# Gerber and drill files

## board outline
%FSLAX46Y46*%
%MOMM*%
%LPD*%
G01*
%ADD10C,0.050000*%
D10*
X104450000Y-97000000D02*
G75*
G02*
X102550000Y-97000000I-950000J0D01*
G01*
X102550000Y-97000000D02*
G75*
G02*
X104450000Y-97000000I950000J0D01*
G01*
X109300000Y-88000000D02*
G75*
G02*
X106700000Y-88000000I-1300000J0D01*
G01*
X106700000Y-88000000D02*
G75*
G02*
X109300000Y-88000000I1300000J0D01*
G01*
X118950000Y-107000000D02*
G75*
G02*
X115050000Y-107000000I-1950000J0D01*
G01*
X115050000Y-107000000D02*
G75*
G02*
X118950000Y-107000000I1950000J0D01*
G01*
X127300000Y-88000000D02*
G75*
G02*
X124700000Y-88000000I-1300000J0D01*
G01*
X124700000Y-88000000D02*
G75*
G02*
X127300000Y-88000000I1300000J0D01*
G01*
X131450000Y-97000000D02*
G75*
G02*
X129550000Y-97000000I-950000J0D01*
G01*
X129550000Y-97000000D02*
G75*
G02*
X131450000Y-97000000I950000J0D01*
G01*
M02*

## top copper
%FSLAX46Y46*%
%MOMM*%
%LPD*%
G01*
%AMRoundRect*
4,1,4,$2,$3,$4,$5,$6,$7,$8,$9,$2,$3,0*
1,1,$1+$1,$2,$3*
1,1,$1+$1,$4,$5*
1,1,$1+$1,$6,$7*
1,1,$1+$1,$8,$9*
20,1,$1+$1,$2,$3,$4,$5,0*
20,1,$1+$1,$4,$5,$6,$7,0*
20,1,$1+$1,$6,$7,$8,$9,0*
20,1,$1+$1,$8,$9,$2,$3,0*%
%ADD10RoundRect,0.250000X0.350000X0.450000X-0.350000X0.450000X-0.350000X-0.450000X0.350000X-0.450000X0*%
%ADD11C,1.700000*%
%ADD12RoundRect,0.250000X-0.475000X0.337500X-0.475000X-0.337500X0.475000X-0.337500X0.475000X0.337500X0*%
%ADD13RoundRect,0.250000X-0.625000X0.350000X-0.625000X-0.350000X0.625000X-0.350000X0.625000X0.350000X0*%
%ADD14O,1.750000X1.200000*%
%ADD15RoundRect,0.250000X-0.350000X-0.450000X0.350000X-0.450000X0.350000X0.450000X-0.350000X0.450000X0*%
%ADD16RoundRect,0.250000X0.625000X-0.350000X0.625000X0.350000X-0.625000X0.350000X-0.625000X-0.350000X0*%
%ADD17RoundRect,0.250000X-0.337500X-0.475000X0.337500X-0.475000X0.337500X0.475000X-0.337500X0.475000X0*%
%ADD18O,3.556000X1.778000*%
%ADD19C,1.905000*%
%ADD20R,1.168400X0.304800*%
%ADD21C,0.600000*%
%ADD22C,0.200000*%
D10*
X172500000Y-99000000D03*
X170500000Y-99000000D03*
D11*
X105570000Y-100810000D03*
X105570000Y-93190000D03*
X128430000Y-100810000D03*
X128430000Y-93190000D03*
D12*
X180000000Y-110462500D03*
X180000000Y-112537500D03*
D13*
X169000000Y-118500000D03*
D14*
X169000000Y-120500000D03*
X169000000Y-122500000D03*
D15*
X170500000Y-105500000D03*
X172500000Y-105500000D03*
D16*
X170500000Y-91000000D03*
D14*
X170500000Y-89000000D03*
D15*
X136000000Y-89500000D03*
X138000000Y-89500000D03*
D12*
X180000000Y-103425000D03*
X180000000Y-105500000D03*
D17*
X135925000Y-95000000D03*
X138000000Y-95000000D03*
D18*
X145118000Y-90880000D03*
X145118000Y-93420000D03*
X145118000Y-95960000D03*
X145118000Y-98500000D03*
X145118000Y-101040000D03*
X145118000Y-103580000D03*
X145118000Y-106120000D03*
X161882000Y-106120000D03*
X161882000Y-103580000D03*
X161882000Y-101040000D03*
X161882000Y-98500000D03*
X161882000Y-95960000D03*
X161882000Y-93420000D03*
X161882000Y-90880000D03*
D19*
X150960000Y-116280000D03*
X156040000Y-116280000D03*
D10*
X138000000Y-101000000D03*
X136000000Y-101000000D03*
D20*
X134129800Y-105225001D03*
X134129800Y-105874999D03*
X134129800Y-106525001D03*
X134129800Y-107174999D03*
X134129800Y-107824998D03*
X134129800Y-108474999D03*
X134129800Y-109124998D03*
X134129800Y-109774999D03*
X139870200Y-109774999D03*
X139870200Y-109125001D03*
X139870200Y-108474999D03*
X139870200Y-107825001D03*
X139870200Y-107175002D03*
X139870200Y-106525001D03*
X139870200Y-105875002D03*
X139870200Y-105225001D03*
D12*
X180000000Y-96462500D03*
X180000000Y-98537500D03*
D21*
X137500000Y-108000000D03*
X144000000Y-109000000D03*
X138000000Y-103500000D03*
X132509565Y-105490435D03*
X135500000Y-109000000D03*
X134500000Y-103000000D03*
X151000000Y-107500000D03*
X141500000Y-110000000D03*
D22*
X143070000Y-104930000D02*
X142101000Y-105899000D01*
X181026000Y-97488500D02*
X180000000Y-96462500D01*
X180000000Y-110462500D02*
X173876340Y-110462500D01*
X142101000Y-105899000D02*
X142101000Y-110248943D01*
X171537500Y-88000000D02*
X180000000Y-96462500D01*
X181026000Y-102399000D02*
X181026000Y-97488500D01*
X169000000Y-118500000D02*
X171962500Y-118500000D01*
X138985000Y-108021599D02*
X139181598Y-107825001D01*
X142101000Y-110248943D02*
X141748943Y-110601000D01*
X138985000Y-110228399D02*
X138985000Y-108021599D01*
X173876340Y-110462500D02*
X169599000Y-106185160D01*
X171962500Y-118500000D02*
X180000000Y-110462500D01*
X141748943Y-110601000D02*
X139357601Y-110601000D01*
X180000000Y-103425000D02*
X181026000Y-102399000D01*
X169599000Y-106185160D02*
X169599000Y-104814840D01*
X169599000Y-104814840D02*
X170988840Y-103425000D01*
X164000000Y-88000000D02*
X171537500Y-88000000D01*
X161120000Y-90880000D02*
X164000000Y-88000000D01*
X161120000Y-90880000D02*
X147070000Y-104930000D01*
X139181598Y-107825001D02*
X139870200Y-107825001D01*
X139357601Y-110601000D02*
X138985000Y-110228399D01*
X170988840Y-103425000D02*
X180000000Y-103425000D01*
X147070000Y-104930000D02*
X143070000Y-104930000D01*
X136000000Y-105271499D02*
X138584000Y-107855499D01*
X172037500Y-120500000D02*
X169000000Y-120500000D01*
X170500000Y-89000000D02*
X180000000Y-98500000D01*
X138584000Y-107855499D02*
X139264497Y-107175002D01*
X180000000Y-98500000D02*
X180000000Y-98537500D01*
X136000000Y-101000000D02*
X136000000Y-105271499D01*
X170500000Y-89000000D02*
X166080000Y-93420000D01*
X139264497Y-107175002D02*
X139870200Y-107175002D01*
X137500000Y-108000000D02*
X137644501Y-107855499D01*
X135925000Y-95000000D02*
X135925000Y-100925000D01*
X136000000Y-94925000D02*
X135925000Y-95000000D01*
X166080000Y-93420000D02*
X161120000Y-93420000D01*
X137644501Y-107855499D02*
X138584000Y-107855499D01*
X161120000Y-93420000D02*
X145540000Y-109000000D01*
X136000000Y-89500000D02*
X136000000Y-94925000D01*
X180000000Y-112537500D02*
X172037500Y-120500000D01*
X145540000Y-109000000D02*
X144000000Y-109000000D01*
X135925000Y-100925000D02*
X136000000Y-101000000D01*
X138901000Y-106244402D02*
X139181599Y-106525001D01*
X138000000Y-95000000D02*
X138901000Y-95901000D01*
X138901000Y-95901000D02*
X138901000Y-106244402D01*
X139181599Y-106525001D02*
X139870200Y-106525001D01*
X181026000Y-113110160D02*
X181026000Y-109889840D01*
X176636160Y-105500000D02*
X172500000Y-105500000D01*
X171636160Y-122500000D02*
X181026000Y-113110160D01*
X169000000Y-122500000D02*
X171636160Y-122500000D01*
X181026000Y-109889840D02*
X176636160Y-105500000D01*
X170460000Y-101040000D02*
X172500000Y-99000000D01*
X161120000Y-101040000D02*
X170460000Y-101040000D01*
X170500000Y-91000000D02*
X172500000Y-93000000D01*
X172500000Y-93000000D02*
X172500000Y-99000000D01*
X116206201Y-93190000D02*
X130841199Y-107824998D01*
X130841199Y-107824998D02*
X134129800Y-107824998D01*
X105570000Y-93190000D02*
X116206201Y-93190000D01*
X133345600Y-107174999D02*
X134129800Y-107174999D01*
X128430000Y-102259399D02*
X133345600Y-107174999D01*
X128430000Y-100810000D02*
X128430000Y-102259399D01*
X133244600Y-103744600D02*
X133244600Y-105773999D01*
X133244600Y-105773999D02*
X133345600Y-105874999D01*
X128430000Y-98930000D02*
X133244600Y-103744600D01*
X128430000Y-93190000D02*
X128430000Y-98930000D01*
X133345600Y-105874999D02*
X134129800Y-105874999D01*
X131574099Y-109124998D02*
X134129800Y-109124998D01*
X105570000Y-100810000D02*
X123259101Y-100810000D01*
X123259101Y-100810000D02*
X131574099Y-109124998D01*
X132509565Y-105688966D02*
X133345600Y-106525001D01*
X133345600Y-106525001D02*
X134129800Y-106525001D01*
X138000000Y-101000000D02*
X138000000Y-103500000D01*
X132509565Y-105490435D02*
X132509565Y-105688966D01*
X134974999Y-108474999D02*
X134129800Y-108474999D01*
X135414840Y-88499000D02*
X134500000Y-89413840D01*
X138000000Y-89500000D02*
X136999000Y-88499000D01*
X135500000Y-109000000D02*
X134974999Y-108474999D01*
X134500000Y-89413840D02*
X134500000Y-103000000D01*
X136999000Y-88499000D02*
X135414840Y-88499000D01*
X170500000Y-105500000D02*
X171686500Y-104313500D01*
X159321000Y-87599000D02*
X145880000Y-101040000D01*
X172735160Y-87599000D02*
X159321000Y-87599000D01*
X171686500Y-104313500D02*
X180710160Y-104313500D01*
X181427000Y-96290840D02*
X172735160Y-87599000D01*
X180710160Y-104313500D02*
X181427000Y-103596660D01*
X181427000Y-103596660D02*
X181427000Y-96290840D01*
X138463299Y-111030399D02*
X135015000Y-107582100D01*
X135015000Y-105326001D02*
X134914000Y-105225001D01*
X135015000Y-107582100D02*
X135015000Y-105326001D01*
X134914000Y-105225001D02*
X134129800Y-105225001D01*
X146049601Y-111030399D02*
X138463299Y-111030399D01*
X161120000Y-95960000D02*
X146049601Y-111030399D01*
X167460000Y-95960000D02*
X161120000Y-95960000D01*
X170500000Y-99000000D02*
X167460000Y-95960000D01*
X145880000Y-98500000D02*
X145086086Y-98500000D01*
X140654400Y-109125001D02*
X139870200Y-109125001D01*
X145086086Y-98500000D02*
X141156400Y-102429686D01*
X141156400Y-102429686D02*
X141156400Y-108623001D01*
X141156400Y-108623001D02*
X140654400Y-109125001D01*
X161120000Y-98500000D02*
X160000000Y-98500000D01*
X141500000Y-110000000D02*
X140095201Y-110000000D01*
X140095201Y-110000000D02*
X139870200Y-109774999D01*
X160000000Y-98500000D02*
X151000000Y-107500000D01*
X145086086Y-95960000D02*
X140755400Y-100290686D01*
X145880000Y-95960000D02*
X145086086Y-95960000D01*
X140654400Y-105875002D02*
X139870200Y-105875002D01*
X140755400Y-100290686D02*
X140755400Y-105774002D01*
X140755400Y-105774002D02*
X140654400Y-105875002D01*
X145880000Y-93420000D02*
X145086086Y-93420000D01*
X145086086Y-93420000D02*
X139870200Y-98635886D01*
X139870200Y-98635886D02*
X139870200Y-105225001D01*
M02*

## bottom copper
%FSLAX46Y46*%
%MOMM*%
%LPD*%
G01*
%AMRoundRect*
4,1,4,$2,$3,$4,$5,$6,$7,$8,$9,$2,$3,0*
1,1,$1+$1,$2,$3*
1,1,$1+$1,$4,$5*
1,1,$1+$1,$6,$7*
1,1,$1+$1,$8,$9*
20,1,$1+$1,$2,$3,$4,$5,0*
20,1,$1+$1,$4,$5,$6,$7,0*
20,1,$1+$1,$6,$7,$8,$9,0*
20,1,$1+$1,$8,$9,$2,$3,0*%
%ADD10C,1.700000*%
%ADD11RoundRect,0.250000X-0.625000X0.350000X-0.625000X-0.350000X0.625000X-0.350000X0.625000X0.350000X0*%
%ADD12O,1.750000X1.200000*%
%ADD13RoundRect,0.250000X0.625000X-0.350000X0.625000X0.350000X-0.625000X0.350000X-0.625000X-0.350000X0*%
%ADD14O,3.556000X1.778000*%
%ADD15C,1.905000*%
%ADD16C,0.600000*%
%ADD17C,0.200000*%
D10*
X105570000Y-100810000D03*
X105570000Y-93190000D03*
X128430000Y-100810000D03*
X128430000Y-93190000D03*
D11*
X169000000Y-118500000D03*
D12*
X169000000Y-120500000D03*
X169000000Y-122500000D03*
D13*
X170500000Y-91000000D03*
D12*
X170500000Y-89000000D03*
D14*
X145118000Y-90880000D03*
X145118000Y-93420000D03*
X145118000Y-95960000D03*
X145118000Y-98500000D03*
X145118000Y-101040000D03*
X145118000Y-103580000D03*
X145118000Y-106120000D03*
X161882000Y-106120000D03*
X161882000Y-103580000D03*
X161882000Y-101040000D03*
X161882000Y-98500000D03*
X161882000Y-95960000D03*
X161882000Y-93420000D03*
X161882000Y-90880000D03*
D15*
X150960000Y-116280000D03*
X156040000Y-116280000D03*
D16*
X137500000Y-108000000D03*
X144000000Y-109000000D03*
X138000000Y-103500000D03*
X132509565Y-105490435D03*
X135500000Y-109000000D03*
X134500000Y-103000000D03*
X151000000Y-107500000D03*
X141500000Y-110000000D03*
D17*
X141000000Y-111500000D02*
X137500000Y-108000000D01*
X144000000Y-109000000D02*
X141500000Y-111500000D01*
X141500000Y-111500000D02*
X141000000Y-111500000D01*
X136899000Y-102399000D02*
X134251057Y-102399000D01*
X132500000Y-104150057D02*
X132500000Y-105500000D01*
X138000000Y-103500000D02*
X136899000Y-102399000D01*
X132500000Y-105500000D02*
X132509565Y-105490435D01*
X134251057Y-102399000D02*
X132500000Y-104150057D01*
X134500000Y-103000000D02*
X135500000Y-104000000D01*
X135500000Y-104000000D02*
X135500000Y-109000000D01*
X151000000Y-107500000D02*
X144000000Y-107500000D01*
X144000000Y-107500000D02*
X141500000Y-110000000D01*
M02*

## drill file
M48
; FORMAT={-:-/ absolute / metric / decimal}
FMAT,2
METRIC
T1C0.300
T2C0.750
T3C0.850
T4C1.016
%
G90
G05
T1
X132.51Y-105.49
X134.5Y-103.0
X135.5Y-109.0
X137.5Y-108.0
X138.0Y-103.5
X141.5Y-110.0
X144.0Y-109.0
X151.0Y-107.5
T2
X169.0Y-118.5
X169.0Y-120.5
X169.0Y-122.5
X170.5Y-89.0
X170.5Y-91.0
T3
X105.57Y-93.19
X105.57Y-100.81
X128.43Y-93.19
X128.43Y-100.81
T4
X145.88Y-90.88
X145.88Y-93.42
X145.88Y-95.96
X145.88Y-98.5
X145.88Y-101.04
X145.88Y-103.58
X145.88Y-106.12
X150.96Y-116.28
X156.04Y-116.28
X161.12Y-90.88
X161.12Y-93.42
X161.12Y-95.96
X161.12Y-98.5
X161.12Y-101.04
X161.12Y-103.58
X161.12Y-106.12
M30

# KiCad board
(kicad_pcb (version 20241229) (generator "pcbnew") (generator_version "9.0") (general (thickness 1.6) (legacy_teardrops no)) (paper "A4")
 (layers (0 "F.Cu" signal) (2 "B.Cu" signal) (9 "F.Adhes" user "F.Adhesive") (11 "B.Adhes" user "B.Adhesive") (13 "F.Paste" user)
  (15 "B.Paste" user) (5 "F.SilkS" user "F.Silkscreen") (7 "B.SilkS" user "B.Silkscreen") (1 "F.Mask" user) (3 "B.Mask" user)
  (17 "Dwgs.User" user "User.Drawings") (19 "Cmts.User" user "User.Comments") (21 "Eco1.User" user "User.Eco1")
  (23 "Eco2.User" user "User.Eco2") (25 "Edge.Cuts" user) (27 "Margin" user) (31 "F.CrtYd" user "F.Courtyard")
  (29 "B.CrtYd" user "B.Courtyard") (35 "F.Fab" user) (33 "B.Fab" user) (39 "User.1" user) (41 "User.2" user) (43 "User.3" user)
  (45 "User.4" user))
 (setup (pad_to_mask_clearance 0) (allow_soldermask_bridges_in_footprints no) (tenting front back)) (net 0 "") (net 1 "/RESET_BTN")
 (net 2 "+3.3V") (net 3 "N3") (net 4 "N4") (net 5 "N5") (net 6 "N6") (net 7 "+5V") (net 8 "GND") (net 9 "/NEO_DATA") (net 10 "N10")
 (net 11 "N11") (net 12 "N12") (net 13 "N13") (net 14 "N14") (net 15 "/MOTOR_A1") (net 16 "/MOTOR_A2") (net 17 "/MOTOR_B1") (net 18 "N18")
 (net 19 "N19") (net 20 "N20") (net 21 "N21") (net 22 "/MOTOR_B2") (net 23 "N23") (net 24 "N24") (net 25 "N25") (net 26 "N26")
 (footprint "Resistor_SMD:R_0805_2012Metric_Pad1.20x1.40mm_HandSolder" (layer "F.Cu") (at 171.5 99 180)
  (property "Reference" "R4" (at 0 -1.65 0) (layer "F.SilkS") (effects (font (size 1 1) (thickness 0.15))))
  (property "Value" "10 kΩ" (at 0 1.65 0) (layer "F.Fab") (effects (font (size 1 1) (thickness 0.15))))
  (pad "1" smd roundrect (at -1 0 180) (size 1.2 1.4) (layers "F.Cu" "F.Mask" "F.Paste") (roundrect_rratio 0.208333) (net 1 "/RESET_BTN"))
  (pad "2" smd roundrect (at 1 0 180) (size 1.2 1.4) (layers "F.Cu" "F.Mask" "F.Paste") (roundrect_rratio 0.208333) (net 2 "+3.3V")))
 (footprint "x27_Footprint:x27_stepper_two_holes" (layer "F.Cu") (at 114.46 86.84 180)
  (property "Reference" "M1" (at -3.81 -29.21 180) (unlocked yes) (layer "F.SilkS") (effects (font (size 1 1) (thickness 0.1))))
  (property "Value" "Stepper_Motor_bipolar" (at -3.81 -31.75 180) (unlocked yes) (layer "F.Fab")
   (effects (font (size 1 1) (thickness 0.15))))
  (fp_circle (center 10.96 -10.16) (end 11.91 -10.16) (stroke (width 0.05) (type default)) (fill no) (layer "Edge.Cuts"))
  (fp_circle (center 6.46 -1.16) (end 7.76 -1.16) (stroke (width 0.05) (type default)) (fill no) (layer "Edge.Cuts"))
  (fp_circle (center -2.54 -20.16) (end -0.59 -20.16) (stroke (width 0.05) (type default)) (fill no) (layer "Edge.Cuts"))
  (fp_circle (center -11.54 -1.16) (end -10.24 -1.16) (stroke (width 0.05) (type default)) (fill no) (layer "Edge.Cuts"))
  (fp_circle (center -16.04 -10.16) (end -15.09 -10.16) (stroke (width 0.05) (type default)) (fill no) (layer "Edge.Cuts"))
  (pad "1" thru_hole circle (at 8.89 -13.97 180) (size 1.7 1.7) (drill 0.85) (layers "*.Cu" "*.Mask") (remove_unused_layers no) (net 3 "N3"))
  (pad "2" thru_hole circle (at 8.89 -6.35 180) (size 1.7 1.7) (drill 0.85) (layers "*.Cu" "*.Mask") (remove_unused_layers no) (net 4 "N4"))
  (pad "3" thru_hole circle (at -13.97 -13.97 180) (size 1.7 1.7) (drill 0.85) (layers "*.Cu" "*.Mask") (remove_unused_layers no)
   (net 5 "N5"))
  (pad "4" thru_hole circle (at -13.97 -6.35 180) (size 1.7 1.7) (drill 0.85) (layers "*.Cu" "*.Mask") (remove_unused_layers no)
   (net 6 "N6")))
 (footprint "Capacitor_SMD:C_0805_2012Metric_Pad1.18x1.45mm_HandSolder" (layer "F.Cu") (at 180 111.5 -90)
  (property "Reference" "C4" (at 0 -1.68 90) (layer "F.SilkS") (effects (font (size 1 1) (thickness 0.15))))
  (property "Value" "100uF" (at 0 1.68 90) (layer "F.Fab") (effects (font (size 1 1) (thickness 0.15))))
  (pad "1" smd roundrect (at -1.0375 0 270) (size 1.175 1.45) (layers "F.Cu" "F.Mask" "F.Paste") (roundrect_rratio 0.212766) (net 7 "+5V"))
  (pad "2" smd roundrect (at 1.0375 0 270) (size 1.175 1.45) (layers "F.Cu" "F.Mask" "F.Paste") (roundrect_rratio 0.212766) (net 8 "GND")))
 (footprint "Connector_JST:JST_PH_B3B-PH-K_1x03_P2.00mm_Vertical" (layer "F.Cu") (at 169 118.5 -90)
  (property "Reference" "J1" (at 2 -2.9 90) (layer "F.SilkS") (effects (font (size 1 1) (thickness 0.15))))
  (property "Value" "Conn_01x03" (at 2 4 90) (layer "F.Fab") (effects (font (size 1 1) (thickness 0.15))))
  (pad "1" thru_hole roundrect (at 0 0 270) (size 1.2 1.75) (drill 0.75) (layers "*.Cu" "*.Mask") (remove_unused_layers no)
   (roundrect_rratio 0.208333) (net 7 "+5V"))
  (pad "2" thru_hole oval (at 2 0 270) (size 1.2 1.75) (drill 0.75) (layers "*.Cu" "*.Mask") (remove_unused_layers no) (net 8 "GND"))
  (pad "3" thru_hole oval (at 4 0 270) (size 1.2 1.75) (drill 0.75) (layers "*.Cu" "*.Mask") (remove_unused_layers no) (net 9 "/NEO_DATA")))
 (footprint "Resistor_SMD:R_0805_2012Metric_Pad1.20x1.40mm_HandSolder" (layer "F.Cu") (at 171.5 105.5)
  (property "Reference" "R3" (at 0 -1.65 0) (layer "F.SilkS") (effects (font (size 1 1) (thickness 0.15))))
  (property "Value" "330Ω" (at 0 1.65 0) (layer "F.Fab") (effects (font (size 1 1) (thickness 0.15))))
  (pad "1" smd roundrect (at -1 0) (size 1.2 1.4) (layers "F.Cu" "F.Mask" "F.Paste") (roundrect_rratio 0.208333) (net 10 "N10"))
  (pad "2" smd roundrect (at 1 0) (size 1.2 1.4) (layers "F.Cu" "F.Mask" "F.Paste") (roundrect_rratio 0.208333) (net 9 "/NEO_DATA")))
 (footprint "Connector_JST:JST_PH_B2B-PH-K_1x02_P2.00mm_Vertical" (layer "F.Cu") (at 170.5 91 90)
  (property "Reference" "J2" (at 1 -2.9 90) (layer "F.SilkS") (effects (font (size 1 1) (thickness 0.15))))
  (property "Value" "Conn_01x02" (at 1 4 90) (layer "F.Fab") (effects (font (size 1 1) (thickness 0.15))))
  (pad "1" thru_hole roundrect (at 0 0 90) (size 1.2 1.75) (drill 0.75) (layers "*.Cu" "*.Mask") (remove_unused_layers no)
   (roundrect_rratio 0.208333) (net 1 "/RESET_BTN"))
  (pad "2" thru_hole oval (at 2 0 90) (size 1.2 1.75) (drill 0.75) (layers "*.Cu" "*.Mask") (remove_unused_layers no) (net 8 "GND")))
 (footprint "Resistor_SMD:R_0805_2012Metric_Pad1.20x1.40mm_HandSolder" (layer "F.Cu") (at 137 89.5)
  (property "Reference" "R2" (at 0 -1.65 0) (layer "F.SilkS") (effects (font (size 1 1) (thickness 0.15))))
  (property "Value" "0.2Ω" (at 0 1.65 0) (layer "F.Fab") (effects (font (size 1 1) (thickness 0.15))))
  (pad "1" smd roundrect (at -1 0) (size 1.2 1.4) (layers "F.Cu" "F.Mask" "F.Paste") (roundrect_rratio 0.208333) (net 8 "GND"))
  (pad "2" smd roundrect (at 1 0) (size 1.2 1.4) (layers "F.Cu" "F.Mask" "F.Paste") (roundrect_rratio 0.208333) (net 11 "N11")))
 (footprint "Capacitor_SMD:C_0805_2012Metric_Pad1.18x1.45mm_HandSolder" (layer "F.Cu") (at 180 104.4625 -90)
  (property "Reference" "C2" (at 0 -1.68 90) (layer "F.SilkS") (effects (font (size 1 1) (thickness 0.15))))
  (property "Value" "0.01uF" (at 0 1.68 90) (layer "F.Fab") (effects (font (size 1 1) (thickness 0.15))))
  (pad "1" smd roundrect (at -1.0375 0 270) (size 1.175 1.45) (layers "F.Cu" "F.Mask" "F.Paste") (roundrect_rratio 0.212766) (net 7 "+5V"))
  (pad "2" smd roundrect (at 1.0375 0 270) (size 1.175 1.45) (layers "F.Cu" "F.Mask" "F.Paste") (roundrect_rratio 0.212766) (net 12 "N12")))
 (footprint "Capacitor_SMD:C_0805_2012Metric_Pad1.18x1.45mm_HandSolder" (layer "F.Cu") (at 136.9625 95)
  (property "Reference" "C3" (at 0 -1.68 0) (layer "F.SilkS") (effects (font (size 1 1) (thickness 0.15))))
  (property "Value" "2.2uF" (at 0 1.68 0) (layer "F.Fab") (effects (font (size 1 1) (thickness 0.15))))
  (pad "1" smd roundrect (at -1.0375 0) (size 1.175 1.45) (layers "F.Cu" "F.Mask" "F.Paste") (roundrect_rratio 0.212766) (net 8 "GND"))
  (pad "2" smd roundrect (at 1.0375 0) (size 1.175 1.45) (layers "F.Cu" "F.Mask" "F.Paste") (roundrect_rratio 0.212766) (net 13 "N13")))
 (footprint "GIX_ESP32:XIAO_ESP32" (layer "F.Cu") (at 153.5 98.5)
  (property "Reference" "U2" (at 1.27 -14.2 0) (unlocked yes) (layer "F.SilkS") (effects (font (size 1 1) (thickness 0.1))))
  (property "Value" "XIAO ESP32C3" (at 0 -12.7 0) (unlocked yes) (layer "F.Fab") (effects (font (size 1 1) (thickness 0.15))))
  (pad "1" thru_hole oval (at -7.62 -7.62) (size 3.556 1.778) (drill 1.016 (offset -0.762 0)) (layers "*.Cu" "*.Mask")
   (remove_unused_layers no) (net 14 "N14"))
  (pad "2" thru_hole oval (at -7.62 -5.08) (size 3.556 1.778) (drill 1.016 (offset -0.762 0)) (layers "*.Cu" "*.Mask")
   (remove_unused_layers no) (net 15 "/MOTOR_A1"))
  (pad "3" thru_hole oval (at -7.62 -2.54) (size 3.556 1.778) (drill 1.016 (offset -0.762 0)) (layers "*.Cu" "*.Mask")
   (remove_unused_layers no) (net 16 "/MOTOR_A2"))
  (pad "4" thru_hole oval (at -7.62 0) (size 3.556 1.778) (drill 1.016 (offset -0.762 0)) (layers "*.Cu" "*.Mask") (remove_unused_layers no)
   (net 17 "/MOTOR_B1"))
  (pad "5" thru_hole oval (at -7.62 2.54) (size 3.556 1.778) (drill 1.016 (offset -0.762 0)) (layers "*.Cu" "*.Mask")
   (remove_unused_layers no) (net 10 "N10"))
  (pad "6" thru_hole oval (at -7.62 5.08) (size 3.556 1.778) (drill 1.016 (offset -0.762 0)) (layers "*.Cu" "*.Mask")
   (remove_unused_layers no) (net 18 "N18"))
  (pad "7" thru_hole oval (at -7.62 7.62) (size 3.556 1.778) (drill 1.016 (offset -0.762 0)) (layers "*.Cu" "*.Mask")
   (remove_unused_layers no) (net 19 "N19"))
  (pad "8" thru_hole oval (at 7.62 7.62) (size 3.556 1.778) (drill 1.016 (offset 0.762 0)) (layers "*.Cu" "*.Mask")
   (remove_unused_layers no) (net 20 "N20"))
  (pad "9" thru_hole oval (at 7.62 5.08) (size 3.556 1.778) (drill 1.016 (offset 0.762 0)) (layers "*.Cu" "*.Mask")
   (remove_unused_layers no) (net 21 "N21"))
  (pad "10" thru_hole oval (at 7.62 2.54) (size 3.556 1.778) (drill 1.016 (offset 0.762 0)) (layers "*.Cu" "*.Mask")
   (remove_unused_layers no) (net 1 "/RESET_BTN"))
  (pad "11" thru_hole oval (at 7.62 0) (size 3.556 1.778) (drill 1.016 (offset 0.762 0)) (layers "*.Cu" "*.Mask") (remove_unused_layers no)
   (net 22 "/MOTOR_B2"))
  (pad "12" thru_hole oval (at 7.62 -2.54) (size 3.556 1.778) (drill 1.016 (offset 0.762 0)) (layers "*.Cu" "*.Mask")
   (remove_unused_layers no) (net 2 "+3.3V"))
  (pad "13" thru_hole oval (at 7.62 -5.08) (size 3.556 1.778) (drill 1.016 (offset 0.762 0)) (layers "*.Cu" "*.Mask")
   (remove_unused_layers no) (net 8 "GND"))
  (pad "14" thru_hole oval (at 7.62 -7.62) (size 3.556 1.778) (drill 1.016 (offset 0.762 0)) (layers "*.Cu" "*.Mask")
   (remove_unused_layers no) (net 7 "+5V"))
  (pad "15" thru_hole circle (at -2.54 17.78) (size 1.905 1.905) (drill 1.016) (layers "*.Cu" "*.Mask") (remove_unused_layers no)
   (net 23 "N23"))
  (pad "16" thru_hole circle (at 2.54 17.78) (size 1.905 1.905) (drill 1.016) (layers "*.Cu" "*.Mask") (remove_unused_layers no)
   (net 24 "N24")))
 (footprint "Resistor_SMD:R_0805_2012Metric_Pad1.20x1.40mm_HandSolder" (layer "F.Cu") (at 137 101 180)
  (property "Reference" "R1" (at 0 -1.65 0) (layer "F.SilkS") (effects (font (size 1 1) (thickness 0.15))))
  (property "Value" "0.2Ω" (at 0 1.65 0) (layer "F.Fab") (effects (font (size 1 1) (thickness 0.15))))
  (pad "1" smd roundrect (at -1 0 180) (size 1.2 1.4) (layers "F.Cu" "F.Mask" "F.Paste") (roundrect_rratio 0.208333) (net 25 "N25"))
  (pad "2" smd roundrect (at 1 0 180) (size 1.2 1.4) (layers "F.Cu" "F.Mask" "F.Paste") (roundrect_rratio 0.208333) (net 8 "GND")))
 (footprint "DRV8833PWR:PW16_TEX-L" (layer "F.Cu") (at 137 107.5)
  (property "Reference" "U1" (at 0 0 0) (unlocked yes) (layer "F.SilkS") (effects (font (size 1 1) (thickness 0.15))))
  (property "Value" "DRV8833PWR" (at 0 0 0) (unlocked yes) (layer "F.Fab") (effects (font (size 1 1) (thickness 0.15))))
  (pad "1" smd rect (at -2.8702 -2.274999) (size 1.1684 0.3048) (layers "F.Cu" "F.Mask" "F.Paste") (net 2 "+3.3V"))
  (pad "2" smd rect (at -2.8702 -1.625001) (size 1.1684 0.3048) (layers "F.Cu" "F.Mask" "F.Paste") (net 6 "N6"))
  (pad "3" smd rect (at -2.8702 -0.974999) (size 1.1684 0.3048) (layers "F.Cu" "F.Mask" "F.Paste") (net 25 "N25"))
  (pad "4" smd rect (at -2.8702 -0.325001) (size 1.1684 0.3048) (layers "F.Cu" "F.Mask" "F.Paste") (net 5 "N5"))
  (pad "5" smd rect (at -2.8702 0.324998) (size 1.1684 0.3048) (layers "F.Cu" "F.Mask" "F.Paste") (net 4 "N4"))
  (pad "6" smd rect (at -2.8702 0.974999) (size 1.1684 0.3048) (layers "F.Cu" "F.Mask" "F.Paste") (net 11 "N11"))
  (pad "7" smd rect (at -2.8702 1.624998) (size 1.1684 0.3048) (layers "F.Cu" "F.Mask" "F.Paste") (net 3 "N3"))
  (pad "8" smd rect (at -2.8702 2.274999) (size 1.1684 0.3048) (layers "F.Cu" "F.Mask" "F.Paste") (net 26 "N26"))
  (pad "9" smd rect (at 2.8702 2.274999) (size 1.1684 0.3048) (layers "F.Cu" "F.Mask" "F.Paste") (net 22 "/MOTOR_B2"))
  (pad "10" smd rect (at 2.8702 1.625001) (size 1.1684 0.3048) (layers "F.Cu" "F.Mask" "F.Paste") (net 17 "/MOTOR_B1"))
  (pad "11" smd rect (at 2.8702 0.974999) (size 1.1684 0.3048) (layers "F.Cu" "F.Mask" "F.Paste") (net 12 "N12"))
  (pad "12" smd rect (at 2.8702 0.325001) (size 1.1684 0.3048) (layers "F.Cu" "F.Mask" "F.Paste") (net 7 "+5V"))
  (pad "13" smd rect (at 2.8702 -0.324998) (size 1.1684 0.3048) (layers "F.Cu" "F.Mask" "F.Paste") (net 8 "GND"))
  (pad "14" smd rect (at 2.8702 -0.974999) (size 1.1684 0.3048) (layers "F.Cu" "F.Mask" "F.Paste") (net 13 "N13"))
  (pad "15" smd rect (at 2.8702 -1.624998) (size 1.1684 0.3048) (layers "F.Cu" "F.Mask" "F.Paste") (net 16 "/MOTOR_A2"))
  (pad "16" smd rect (at 2.8702 -2.274999) (size 1.1684 0.3048) (layers "F.Cu" "F.Mask" "F.Paste") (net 15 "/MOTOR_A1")))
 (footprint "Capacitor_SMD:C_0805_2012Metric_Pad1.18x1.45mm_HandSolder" (layer "F.Cu") (at 180 97.5 -90)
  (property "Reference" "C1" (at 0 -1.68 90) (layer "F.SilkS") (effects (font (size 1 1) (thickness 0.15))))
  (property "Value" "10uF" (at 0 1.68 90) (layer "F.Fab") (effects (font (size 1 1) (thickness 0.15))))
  (pad "1" smd roundrect (at -1.0375 0 270) (size 1.175 1.45) (layers "F.Cu" "F.Mask" "F.Paste") (roundrect_rratio 0.212766) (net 7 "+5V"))
  (pad "2" smd roundrect (at 1.0375 0 270) (size 1.175 1.45) (layers "F.Cu" "F.Mask" "F.Paste") (roundrect_rratio 0.212766) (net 8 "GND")))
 (segment (start 143.07 104.93) (end 142.101 105.899) (width 0.2) (layer "F.Cu") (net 7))
 (segment (start 181.026 97.4885) (end 180 96.4625) (width 0.2) (layer "F.Cu") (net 7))
 (segment (start 180 110.4625) (end 173.87634 110.4625) (width 0.2) (layer "F.Cu") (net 7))
 (segment (start 142.101 105.899) (end 142.101 110.248943) (width 0.2) (layer "F.Cu") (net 7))
 (segment (start 171.5375 88) (end 180 96.4625) (width 0.2) (layer "F.Cu") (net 7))
 (segment (start 181.026 102.399) (end 181.026 97.4885) (width 0.2) (layer "F.Cu") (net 7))
 (segment (start 169 118.5) (end 171.9625 118.5) (width 0.2) (layer "F.Cu") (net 7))
 (segment (start 138.985 108.021599) (end 139.181598 107.825001) (width 0.2) (layer "F.Cu") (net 7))
 (segment (start 142.101 110.248943) (end 141.748943 110.601) (width 0.2) (layer "F.Cu") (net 7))
 (segment (start 138.985 110.228399) (end 138.985 108.021599) (width 0.2) (layer "F.Cu") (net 7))
 (segment (start 173.87634 110.4625) (end 169.599 106.18516) (width 0.2) (layer "F.Cu") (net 7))
 (segment (start 171.9625 118.5) (end 180 110.4625) (width 0.2) (layer "F.Cu") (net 7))
 (segment (start 141.748943 110.601) (end 139.357601 110.601) (width 0.2) (layer "F.Cu") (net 7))
 (segment (start 180 103.425) (end 181.026 102.399) (width 0.2) (layer "F.Cu") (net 7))
 (segment (start 169.599 106.18516) (end 169.599 104.81484) (width 0.2) (layer "F.Cu") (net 7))
 (segment (start 169.599 104.81484) (end 170.98884 103.425) (width 0.2) (layer "F.Cu") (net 7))
 (segment (start 164 88) (end 171.5375 88) (width 0.2) (layer "F.Cu") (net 7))
 (segment (start 161.12 90.88) (end 164 88) (width 0.2) (layer "F.Cu") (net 7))
 (segment (start 161.12 90.88) (end 147.07 104.93) (width 0.2) (layer "F.Cu") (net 7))
 (segment (start 139.181598 107.825001) (end 139.8702 107.825001) (width 0.2) (layer "F.Cu") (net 7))
 (segment (start 139.357601 110.601) (end 138.985 110.228399) (width 0.2) (layer "F.Cu") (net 7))
 (segment (start 170.98884 103.425) (end 180 103.425) (width 0.2) (layer "F.Cu") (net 7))
 (segment (start 147.07 104.93) (end 143.07 104.93) (width 0.2) (layer "F.Cu") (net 7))
 (segment (start 136 105.271499) (end 138.584 107.855499) (width 0.2) (layer "F.Cu") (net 8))
 (segment (start 172.0375 120.5) (end 169 120.5) (width 0.2) (layer "F.Cu") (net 8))
 (segment (start 170.5 89) (end 180 98.5) (width 0.2) (layer "F.Cu") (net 8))
 (segment (start 138.584 107.855499) (end 139.264497 107.175002) (width 0.2) (layer "F.Cu") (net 8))
 (segment (start 180 98.5) (end 180 98.5375) (width 0.2) (layer "F.Cu") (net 8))
 (segment (start 136 101) (end 136 105.271499) (width 0.2) (layer "F.Cu") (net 8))
 (segment (start 170.5 89) (end 166.08 93.42) (width 0.2) (layer "F.Cu") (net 8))
 (segment (start 139.264497 107.175002) (end 139.8702 107.175002) (width 0.2) (layer "F.Cu") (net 8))
 (segment (start 137.5 108) (end 137.644501 107.855499) (width 0.2) (layer "F.Cu") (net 8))
 (segment (start 135.925 95) (end 135.925 100.925) (width 0.2) (layer "F.Cu") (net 8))
 (segment (start 136 94.925) (end 135.925 95) (width 0.2) (layer "F.Cu") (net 8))
 (segment (start 166.08 93.42) (end 161.12 93.42) (width 0.2) (layer "F.Cu") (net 8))
 (segment (start 137.644501 107.855499) (end 138.584 107.855499) (width 0.2) (layer "F.Cu") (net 8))
 (segment (start 161.12 93.42) (end 145.54 109) (width 0.2) (layer "F.Cu") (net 8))
 (segment (start 136 89.5) (end 136 94.925) (width 0.2) (layer "F.Cu") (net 8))
 (segment (start 180 112.5375) (end 172.0375 120.5) (width 0.2) (layer "F.Cu") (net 8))
 (segment (start 145.54 109) (end 144 109) (width 0.2) (layer "F.Cu") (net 8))
 (segment (start 135.925 100.925) (end 136 101) (width 0.2) (layer "F.Cu") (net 8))
 (via (at 137.5 108) (size 0.6) (drill 0.3) (layers "F.Cu" "B.Cu") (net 8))
 (via (at 144 109) (size 0.6) (drill 0.3) (layers "F.Cu" "B.Cu") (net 8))
 (segment (start 141 111.5) (end 137.5 108) (width 0.2) (layer "B.Cu") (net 8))
 (segment (start 144 109) (end 141.5 111.5) (width 0.2) (layer "B.Cu") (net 8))
 (segment (start 141.5 111.5) (end 141 111.5) (width 0.2) (layer "B.Cu") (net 8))
 (segment (start 138.901 106.244402) (end 139.181599 106.525001) (width 0.2) (layer "F.Cu") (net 13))
 (segment (start 138 95) (end 138.901 95.901) (width 0.2) (layer "F.Cu") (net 13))
 (segment (start 138.901 95.901) (end 138.901 106.244402) (width 0.2) (layer "F.Cu") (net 13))
 (segment (start 139.181599 106.525001) (end 139.8702 106.525001) (width 0.2) (layer "F.Cu") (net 13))
 (segment (start 181.026 113.11016) (end 181.026 109.88984) (width 0.2) (layer "F.Cu") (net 9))
 (segment (start 176.63616 105.5) (end 172.5 105.5) (width 0.2) (layer "F.Cu") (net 9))
 (segment (start 171.63616 122.5) (end 181.026 113.11016) (width 0.2) (layer "F.Cu") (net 9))
 (segment (start 169 122.5) (end 171.63616 122.5) (width 0.2) (layer "F.Cu") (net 9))
 (segment (start 181.026 109.88984) (end 176.63616 105.5) (width 0.2) (layer "F.Cu") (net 9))
 (segment (start 170.46 101.04) (end 172.5 99) (width 0.2) (layer "F.Cu") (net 1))
 (segment (start 161.12 101.04) (end 170.46 101.04) (width 0.2) (layer "F.Cu") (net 1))
 (segment (start 170.5 91) (end 172.5 93) (width 0.2) (layer "F.Cu") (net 1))
 (segment (start 172.5 93) (end 172.5 99) (width 0.2) (layer "F.Cu") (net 1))
 (segment (start 116.206201 93.19) (end 130.841199 107.824998) (width 0.2) (layer "F.Cu") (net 4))
 (segment (start 130.841199 107.824998) (end 134.1298 107.824998) (width 0.2) (layer "F.Cu") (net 4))
 (segment (start 105.57 93.19) (end 116.206201 93.19) (width 0.2) (layer "F.Cu") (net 4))
 (segment (start 133.3456 107.174999) (end 134.1298 107.174999) (width 0.2) (layer "F.Cu") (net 5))
 (segment (start 128.43 102.259399) (end 133.3456 107.174999) (width 0.2) (layer "F.Cu") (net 5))
 (segment (start 128.43 100.81) (end 128.43 102.259399) (width 0.2) (layer "F.Cu") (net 5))
 (segment (start 133.2446 103.7446) (end 133.2446 105.773999) (width 0.2) (layer "F.Cu") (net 6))
 (segment (start 133.2446 105.773999) (end 133.3456 105.874999) (width 0.2) (layer "F.Cu") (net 6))
 (segment (start 128.43 98.93) (end 133.2446 103.7446) (width 0.2) (layer "F.Cu") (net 6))
 (segment (start 128.43 93.19) (end 128.43 98.93) (width 0.2) (layer "F.Cu") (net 6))
 (segment (start 133.3456 105.874999) (end 134.1298 105.874999) (width 0.2) (layer "F.Cu") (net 6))
 (segment (start 131.574099 109.124998) (end 134.1298 109.124998) (width 0.2) (layer "F.Cu") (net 3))
 (segment (start 105.57 100.81) (end 123.259101 100.81) (width 0.2) (layer "F.Cu") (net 3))
 (segment (start 123.259101 100.81) (end 131.574099 109.124998) (width 0.2) (layer "F.Cu") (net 3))
 (segment (start 132.509565 105.688966) (end 133.3456 106.525001) (width 0.2) (layer "F.Cu") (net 25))
 (segment (start 133.3456 106.525001) (end 134.1298 106.525001) (width 0.2) (layer "F.Cu") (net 25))
 (segment (start 138 101) (end 138 103.5) (width 0.2) (layer "F.Cu") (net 25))
 (segment (start 132.509565 105.490435) (end 132.509565 105.688966) (width 0.2) (layer "F.Cu") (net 25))
 (via (at 138 103.5) (size 0.6) (drill 0.3) (layers "F.Cu" "B.Cu") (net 25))
 (via (at 132.509565 105.490435) (size 0.6) (drill 0.3) (layers "F.Cu" "B.Cu") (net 25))
 (segment (start 136.899 102.399) (end 134.251057 102.399) (width 0.2) (layer "B.Cu") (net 25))
 (segment (start 132.5 104.150057) (end 132.5 105.5) (width 0.2) (layer "B.Cu") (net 25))
 (segment (start 138 103.5) (end 136.899 102.399) (width 0.2) (layer "B.Cu") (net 25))
 (segment (start 132.5 105.5) (end 132.509565 105.490435) (width 0.2) (layer "B.Cu") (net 25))
 (segment (start 134.251057 102.399) (end 132.5 104.150057) (width 0.2) (layer "B.Cu") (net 25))
 (segment (start 134.974999 108.474999) (end 134.1298 108.474999) (width 0.2) (layer "F.Cu") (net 11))
 (segment (start 135.41484 88.499) (end 134.5 89.41384) (width 0.2) (layer "F.Cu") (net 11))
 (segment (start 138 89.5) (end 136.999 88.499) (width 0.2) (layer "F.Cu") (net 11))
 (segment (start 135.5 109) (end 134.974999 108.474999) (width 0.2) (layer "F.Cu") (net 11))
 (segment (start 134.5 89.41384) (end 134.5 103) (width 0.2) (layer "F.Cu") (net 11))
 (segment (start 136.999 88.499) (end 135.41484 88.499) (width 0.2) (layer "F.Cu") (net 11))
 (via (at 135.5 109) (size 0.6) (drill 0.3) (layers "F.Cu" "B.Cu") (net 11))
 (via (at 134.5 103) (size 0.6) (drill 0.3) (layers "F.Cu" "B.Cu") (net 11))
 (segment (start 134.5 103) (end 135.5 104) (width 0.2) (layer "B.Cu") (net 11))
 (segment (start 135.5 104) (end 135.5 109) (width 0.2) (layer "B.Cu") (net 11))
 (segment (start 170.5 105.5) (end 171.6865 104.3135) (width 0.2) (layer "F.Cu") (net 10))
 (segment (start 159.321 87.599) (end 145.88 101.04) (width 0.2) (layer "F.Cu") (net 10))
 (segment (start 172.73516 87.599) (end 159.321 87.599) (width 0.2) (layer "F.Cu") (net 10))
 (segment (start 171.6865 104.3135) (end 180.71016 104.3135) (width 0.2) (layer "F.Cu") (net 10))
 (segment (start 181.427 96.29084) (end 172.73516 87.599) (width 0.2) (layer "F.Cu") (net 10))
 (segment (start 180.71016 104.3135) (end 181.427 103.59666) (width 0.2) (layer "F.Cu") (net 10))
 (segment (start 181.427 103.59666) (end 181.427 96.29084) (width 0.2) (layer "F.Cu") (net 10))
 (segment (start 138.463299 111.030399) (end 135.015 107.5821) (width 0.2) (layer "F.Cu") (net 2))
 (segment (start 135.015 105.326001) (end 134.914 105.225001) (width 0.2) (layer "F.Cu") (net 2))
 (segment (start 135.015 107.5821) (end 135.015 105.326001) (width 0.2) (layer "F.Cu") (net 2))
 (segment (start 134.914 105.225001) (end 134.1298 105.225001) (width 0.2) (layer "F.Cu") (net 2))
 (segment (start 146.049601 111.030399) (end 138.463299 111.030399) (width 0.2) (layer "F.Cu") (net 2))
 (segment (start 161.12 95.96) (end 146.049601 111.030399) (width 0.2) (layer "F.Cu") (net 2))
 (segment (start 167.46 95.96) (end 161.12 95.96) (width 0.2) (layer "F.Cu") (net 2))
 (segment (start 170.5 99) (end 167.46 95.96) (width 0.2) (layer "F.Cu") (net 2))
 (segment (start 145.88 98.5) (end 145.086086 98.5) (width 0.2) (layer "F.Cu") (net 17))
 (segment (start 140.6544 109.125001) (end 139.8702 109.125001) (width 0.2) (layer "F.Cu") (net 17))
 (segment (start 145.086086 98.5) (end 141.1564 102.429686) (width 0.2) (layer "F.Cu") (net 17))
 (segment (start 141.1564 102.429686) (end 141.1564 108.623001) (width 0.2) (layer "F.Cu") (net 17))
 (segment (start 141.1564 108.623001) (end 140.6544 109.125001) (width 0.2) (layer "F.Cu") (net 17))
 (segment (start 161.12 98.5) (end 160 98.5) (width 0.2) (layer "F.Cu") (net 22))
 (segment (start 141.5 110) (end 140.095201 110) (width 0.2) (layer "F.Cu") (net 22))
 (segment (start 140.095201 110) (end 139.8702 109.774999) (width 0.2) (layer "F.Cu") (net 22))
 (segment (start 160 98.5) (end 151 107.5) (width 0.2) (layer "F.Cu") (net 22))
 (via (at 151 107.5) (size 0.6) (drill 0.3) (layers "F.Cu" "B.Cu") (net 22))
 (via (at 141.5 110) (size 0.6) (drill 0.3) (layers "F.Cu" "B.Cu") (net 22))
 (segment (start 151 107.5) (end 144 107.5) (width 0.2) (layer "B.Cu") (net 22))
 (segment (start 144 107.5) (end 141.5 110) (width 0.2) (layer "B.Cu") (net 22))
 (segment (start 145.086086 95.96) (end 140.7554 100.290686) (width 0.2) (layer "F.Cu") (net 16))
 (segment (start 145.88 95.96) (end 145.086086 95.96) (width 0.2) (layer "F.Cu") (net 16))
 (segment (start 140.6544 105.875002) (end 139.8702 105.875002) (width 0.2) (layer "F.Cu") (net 16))
 (segment (start 140.7554 100.290686) (end 140.7554 105.774002) (width 0.2) (layer "F.Cu") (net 16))
 (segment (start 140.7554 105.774002) (end 140.6544 105.875002) (width 0.2) (layer "F.Cu") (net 16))
 (segment (start 145.88 93.42) (end 145.086086 93.42) (width 0.2) (layer "F.Cu") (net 15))
 (segment (start 145.086086 93.42) (end 139.8702 98.635886) (width 0.2) (layer "F.Cu") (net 15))
 (segment (start 139.8702 98.635886) (end 139.8702 105.225001) (width 0.2) (layer "F.Cu") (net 15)))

